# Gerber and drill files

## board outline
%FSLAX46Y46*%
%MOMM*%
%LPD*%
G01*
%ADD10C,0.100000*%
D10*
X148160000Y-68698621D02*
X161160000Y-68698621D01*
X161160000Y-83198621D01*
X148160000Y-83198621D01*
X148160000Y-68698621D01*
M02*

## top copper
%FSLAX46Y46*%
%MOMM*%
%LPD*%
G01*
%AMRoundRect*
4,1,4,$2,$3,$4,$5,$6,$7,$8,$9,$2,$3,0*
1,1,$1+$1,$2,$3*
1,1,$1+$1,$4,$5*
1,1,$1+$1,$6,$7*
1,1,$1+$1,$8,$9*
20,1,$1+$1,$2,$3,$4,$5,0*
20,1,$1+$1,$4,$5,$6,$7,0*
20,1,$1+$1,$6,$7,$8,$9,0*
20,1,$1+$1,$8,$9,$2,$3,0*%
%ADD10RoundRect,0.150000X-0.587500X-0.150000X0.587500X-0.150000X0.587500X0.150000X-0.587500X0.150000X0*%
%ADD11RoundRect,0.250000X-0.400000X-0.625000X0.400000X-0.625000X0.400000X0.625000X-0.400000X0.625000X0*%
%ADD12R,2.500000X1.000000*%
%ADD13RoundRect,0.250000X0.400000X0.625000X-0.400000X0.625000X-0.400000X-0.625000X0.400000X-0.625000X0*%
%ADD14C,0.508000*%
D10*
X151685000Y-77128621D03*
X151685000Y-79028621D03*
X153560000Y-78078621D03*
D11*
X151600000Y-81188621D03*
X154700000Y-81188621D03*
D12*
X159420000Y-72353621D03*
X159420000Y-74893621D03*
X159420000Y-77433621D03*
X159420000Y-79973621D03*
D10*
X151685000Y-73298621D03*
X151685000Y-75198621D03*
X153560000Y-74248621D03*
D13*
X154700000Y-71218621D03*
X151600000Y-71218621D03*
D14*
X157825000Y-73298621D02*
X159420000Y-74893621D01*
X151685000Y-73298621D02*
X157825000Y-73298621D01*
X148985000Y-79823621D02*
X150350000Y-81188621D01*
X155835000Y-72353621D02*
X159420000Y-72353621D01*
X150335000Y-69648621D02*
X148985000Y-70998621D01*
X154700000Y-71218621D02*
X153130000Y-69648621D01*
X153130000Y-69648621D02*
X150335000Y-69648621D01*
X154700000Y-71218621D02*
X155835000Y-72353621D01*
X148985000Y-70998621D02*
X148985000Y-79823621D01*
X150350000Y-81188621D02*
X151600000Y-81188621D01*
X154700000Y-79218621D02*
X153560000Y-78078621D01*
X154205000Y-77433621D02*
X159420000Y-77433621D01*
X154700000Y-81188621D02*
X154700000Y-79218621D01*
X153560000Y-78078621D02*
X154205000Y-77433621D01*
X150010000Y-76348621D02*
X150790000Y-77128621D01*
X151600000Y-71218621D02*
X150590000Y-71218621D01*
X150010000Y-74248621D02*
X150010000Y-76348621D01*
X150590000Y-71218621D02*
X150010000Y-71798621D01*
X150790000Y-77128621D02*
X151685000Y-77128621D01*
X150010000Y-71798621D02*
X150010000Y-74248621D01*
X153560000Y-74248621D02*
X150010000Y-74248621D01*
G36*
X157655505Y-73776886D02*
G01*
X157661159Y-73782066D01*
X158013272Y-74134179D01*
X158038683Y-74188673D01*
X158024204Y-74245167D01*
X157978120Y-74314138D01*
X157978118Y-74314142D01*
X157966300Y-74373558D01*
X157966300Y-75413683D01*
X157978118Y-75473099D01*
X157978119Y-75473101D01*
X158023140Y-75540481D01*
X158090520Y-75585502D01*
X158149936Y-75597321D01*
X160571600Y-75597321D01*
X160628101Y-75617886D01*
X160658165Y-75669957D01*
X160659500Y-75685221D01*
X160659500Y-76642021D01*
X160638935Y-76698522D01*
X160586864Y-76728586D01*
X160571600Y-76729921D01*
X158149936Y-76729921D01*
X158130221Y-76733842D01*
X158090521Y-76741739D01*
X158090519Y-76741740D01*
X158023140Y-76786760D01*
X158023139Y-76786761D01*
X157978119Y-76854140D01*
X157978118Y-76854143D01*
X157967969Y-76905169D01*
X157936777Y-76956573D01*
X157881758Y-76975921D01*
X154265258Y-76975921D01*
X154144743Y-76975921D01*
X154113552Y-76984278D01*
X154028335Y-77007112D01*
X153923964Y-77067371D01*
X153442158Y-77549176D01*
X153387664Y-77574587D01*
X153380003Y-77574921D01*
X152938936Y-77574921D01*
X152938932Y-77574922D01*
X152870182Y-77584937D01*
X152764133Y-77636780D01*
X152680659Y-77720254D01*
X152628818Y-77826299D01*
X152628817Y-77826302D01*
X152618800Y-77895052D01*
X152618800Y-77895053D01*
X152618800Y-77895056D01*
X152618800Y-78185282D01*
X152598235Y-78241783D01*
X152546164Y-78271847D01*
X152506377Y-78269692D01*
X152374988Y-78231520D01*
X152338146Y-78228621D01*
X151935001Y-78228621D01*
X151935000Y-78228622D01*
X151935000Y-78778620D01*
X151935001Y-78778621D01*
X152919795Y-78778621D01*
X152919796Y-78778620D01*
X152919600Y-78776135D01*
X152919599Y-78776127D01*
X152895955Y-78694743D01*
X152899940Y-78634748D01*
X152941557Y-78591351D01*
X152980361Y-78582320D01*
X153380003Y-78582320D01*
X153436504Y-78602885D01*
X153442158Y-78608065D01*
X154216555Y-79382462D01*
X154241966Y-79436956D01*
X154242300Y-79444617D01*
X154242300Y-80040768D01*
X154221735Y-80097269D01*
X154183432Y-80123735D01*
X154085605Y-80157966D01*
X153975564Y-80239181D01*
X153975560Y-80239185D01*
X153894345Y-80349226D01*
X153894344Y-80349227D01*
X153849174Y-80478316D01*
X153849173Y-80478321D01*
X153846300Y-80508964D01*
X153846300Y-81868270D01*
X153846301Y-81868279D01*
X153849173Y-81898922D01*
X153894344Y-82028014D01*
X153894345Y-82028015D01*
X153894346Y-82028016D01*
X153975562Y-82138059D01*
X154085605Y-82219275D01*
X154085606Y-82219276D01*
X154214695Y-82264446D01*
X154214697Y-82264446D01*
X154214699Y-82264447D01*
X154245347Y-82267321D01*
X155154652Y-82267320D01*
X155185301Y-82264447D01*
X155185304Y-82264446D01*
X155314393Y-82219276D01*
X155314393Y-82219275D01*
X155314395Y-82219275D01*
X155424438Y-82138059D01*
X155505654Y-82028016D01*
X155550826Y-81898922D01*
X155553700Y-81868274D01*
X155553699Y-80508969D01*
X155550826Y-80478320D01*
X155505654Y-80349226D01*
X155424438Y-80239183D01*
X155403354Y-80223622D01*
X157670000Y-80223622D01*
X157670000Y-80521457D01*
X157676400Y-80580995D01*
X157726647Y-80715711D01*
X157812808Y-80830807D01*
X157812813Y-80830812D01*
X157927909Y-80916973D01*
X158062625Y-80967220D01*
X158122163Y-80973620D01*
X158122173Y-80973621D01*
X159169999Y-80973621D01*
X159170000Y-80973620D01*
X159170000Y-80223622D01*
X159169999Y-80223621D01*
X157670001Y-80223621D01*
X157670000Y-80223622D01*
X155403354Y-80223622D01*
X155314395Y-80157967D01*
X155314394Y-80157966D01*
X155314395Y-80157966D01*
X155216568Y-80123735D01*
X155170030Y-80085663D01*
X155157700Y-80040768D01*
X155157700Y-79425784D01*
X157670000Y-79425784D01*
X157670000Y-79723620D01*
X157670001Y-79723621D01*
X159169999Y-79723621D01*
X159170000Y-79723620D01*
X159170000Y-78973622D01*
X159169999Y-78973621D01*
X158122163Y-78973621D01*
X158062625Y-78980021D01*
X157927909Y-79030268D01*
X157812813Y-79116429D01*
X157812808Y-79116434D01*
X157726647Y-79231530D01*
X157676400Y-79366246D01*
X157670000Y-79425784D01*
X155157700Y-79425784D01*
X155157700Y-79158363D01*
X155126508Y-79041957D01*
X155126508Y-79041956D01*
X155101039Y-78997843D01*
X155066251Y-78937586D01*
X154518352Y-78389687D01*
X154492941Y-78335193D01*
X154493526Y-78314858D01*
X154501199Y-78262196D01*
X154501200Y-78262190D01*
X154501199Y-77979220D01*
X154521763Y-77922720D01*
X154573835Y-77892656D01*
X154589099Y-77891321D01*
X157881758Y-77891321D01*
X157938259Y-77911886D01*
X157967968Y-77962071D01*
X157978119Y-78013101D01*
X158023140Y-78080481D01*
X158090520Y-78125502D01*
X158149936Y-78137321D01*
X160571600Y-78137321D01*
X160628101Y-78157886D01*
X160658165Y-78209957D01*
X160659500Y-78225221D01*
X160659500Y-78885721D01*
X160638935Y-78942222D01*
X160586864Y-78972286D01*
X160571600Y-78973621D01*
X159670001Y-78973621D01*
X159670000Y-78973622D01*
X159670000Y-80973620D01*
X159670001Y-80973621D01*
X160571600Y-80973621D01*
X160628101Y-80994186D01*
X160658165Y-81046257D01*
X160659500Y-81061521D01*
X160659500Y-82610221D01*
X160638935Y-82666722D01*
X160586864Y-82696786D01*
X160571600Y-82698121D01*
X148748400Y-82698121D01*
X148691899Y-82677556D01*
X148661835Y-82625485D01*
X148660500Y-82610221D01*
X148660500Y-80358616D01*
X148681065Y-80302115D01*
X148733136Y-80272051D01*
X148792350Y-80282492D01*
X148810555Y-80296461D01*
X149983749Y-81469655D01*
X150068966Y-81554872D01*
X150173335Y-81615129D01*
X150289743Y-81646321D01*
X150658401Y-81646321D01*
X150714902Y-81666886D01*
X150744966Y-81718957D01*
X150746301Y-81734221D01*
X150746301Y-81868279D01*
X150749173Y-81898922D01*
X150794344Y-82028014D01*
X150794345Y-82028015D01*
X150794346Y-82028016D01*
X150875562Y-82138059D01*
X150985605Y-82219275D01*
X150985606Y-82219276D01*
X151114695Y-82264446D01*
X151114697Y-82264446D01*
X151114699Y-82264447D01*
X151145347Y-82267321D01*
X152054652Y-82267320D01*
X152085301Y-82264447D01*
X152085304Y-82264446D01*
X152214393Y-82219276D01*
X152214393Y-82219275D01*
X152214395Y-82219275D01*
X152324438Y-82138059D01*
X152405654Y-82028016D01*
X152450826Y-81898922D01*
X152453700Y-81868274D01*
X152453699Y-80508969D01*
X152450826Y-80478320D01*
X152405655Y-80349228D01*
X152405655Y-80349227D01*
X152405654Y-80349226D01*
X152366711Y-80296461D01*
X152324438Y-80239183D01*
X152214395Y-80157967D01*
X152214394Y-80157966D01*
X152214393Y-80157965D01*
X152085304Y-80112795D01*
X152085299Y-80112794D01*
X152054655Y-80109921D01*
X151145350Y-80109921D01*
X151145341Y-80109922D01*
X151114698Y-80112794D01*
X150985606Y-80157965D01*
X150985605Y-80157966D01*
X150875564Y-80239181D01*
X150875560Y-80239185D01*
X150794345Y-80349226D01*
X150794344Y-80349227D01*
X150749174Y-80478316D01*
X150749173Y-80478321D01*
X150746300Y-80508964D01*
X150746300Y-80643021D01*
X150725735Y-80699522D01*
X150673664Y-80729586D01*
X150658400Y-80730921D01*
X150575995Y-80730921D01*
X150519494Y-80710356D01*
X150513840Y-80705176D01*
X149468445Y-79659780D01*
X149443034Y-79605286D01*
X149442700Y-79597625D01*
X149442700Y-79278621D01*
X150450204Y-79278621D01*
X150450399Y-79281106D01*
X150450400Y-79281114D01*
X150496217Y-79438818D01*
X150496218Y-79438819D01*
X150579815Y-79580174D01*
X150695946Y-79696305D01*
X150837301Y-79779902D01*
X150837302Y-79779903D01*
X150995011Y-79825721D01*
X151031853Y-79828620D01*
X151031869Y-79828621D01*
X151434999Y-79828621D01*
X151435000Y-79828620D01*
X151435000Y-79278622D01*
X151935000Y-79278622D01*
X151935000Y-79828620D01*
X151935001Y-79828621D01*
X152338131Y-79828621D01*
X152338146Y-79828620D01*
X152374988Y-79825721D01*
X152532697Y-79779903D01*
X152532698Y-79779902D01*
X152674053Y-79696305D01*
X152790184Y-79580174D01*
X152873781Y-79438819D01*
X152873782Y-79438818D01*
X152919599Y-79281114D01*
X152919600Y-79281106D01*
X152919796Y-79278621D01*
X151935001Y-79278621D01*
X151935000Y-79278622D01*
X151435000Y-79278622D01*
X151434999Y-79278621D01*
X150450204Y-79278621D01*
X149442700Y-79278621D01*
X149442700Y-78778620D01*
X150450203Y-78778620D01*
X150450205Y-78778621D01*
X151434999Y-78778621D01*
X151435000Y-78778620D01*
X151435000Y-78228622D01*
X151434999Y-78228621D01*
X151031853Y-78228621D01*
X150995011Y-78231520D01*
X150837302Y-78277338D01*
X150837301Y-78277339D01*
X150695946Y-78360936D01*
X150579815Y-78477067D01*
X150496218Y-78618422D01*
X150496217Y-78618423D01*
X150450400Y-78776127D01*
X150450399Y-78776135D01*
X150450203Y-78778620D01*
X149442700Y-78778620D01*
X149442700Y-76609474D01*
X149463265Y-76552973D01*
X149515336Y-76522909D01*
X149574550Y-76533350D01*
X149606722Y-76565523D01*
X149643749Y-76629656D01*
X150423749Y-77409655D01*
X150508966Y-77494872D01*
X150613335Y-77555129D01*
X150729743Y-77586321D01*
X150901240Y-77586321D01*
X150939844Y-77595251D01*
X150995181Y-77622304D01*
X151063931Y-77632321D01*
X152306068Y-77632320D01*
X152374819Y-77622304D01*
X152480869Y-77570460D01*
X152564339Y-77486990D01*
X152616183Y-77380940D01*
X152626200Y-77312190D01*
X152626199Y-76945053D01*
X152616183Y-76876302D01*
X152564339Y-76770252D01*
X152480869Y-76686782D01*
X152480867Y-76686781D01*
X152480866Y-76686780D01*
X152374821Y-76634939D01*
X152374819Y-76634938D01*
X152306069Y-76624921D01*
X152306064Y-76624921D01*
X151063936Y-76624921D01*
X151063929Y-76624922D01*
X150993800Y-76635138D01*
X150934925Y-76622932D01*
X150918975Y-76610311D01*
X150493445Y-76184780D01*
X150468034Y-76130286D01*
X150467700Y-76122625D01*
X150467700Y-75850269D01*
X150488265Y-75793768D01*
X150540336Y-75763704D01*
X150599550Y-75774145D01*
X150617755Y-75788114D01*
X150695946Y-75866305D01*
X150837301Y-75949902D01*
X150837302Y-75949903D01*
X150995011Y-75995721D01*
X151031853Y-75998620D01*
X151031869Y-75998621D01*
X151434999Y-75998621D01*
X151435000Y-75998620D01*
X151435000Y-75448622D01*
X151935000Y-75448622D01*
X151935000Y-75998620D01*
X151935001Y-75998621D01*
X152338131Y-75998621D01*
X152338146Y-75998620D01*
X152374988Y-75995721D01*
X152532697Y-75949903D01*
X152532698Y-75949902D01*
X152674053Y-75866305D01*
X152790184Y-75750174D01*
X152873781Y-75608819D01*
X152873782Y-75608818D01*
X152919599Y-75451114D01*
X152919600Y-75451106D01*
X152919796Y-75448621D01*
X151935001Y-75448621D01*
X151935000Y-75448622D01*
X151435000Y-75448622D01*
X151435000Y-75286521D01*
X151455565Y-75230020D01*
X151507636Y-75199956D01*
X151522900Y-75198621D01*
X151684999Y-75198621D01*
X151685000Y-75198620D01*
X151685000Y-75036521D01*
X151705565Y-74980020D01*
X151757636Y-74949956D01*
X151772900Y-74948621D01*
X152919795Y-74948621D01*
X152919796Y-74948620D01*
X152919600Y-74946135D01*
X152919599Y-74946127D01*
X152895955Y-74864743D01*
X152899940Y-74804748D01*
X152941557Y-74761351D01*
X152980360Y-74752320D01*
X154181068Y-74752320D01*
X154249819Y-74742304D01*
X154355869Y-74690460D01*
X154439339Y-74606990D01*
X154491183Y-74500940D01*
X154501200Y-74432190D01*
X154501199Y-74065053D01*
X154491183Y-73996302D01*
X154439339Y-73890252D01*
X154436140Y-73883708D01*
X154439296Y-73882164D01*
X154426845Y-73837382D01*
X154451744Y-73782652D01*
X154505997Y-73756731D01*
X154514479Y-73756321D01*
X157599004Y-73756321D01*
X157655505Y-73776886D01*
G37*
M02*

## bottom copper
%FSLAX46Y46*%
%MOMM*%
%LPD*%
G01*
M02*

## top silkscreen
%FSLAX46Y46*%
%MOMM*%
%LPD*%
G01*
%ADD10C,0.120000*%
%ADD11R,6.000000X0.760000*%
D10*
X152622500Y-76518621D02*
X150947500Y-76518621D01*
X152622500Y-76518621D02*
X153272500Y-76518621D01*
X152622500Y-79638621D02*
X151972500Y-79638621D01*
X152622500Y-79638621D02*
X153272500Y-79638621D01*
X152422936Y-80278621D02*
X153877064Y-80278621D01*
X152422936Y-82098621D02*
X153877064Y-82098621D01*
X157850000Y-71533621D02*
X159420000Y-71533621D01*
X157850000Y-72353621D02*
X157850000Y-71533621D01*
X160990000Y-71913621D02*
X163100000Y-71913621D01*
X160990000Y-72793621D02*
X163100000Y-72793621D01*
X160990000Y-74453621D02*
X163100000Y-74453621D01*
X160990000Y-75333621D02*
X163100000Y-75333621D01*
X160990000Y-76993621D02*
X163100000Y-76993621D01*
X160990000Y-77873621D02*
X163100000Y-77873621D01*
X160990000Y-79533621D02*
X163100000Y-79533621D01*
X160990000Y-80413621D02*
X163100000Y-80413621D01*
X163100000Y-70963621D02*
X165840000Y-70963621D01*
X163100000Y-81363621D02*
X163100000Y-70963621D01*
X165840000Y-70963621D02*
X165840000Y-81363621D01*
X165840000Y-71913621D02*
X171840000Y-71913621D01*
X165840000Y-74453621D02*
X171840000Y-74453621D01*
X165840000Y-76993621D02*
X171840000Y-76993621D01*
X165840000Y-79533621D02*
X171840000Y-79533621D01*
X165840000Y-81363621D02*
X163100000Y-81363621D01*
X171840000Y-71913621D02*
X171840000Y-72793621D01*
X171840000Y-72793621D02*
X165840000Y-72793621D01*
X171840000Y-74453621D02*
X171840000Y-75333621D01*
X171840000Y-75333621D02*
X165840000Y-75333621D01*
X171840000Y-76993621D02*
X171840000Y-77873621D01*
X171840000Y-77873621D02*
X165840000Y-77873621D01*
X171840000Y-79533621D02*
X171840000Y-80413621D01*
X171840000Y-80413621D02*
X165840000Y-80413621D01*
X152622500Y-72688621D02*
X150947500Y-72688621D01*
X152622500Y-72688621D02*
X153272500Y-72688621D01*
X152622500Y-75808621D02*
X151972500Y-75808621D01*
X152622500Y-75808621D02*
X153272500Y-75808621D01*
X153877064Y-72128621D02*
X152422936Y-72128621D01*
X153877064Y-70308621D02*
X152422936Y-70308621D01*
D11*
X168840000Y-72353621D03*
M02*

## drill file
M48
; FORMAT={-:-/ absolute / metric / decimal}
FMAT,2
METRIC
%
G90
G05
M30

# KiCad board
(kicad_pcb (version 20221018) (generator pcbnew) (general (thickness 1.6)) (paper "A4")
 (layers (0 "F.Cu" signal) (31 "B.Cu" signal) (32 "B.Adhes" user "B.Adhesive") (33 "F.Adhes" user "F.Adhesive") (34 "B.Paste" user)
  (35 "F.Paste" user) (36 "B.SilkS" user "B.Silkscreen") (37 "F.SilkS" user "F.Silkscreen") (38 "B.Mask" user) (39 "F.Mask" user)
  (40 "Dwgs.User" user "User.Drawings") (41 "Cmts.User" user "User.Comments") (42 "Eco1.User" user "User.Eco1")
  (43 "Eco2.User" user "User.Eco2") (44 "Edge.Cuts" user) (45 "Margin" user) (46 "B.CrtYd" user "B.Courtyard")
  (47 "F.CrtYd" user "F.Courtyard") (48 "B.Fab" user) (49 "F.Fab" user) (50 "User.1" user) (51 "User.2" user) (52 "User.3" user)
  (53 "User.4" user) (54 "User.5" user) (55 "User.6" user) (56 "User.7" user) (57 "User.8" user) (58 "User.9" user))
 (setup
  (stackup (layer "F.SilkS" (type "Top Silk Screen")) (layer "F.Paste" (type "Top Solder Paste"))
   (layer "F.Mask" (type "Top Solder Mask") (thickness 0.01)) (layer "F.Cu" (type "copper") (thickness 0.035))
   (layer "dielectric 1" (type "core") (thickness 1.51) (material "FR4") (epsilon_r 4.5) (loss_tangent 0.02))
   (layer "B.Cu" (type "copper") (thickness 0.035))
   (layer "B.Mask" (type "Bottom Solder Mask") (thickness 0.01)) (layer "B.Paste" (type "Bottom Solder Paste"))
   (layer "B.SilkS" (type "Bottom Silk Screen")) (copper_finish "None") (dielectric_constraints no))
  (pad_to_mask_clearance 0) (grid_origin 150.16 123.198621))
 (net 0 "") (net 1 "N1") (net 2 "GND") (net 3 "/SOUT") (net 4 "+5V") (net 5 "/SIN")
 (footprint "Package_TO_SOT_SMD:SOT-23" (layer "F.Cu") (at 152.6225 78.078621)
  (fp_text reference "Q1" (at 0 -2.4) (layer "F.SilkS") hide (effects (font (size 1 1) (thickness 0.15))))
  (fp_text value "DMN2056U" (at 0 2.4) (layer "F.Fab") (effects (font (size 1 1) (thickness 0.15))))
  (fp_line (start 0 -1.56) (end -1.675 -1.56) (stroke (width 0.12) (type solid)) (layer "F.SilkS"))
  (fp_line (start 0 -1.56) (end 0.65 -1.56) (stroke (width 0.12) (type solid)) (layer "F.SilkS"))
  (fp_line (start 0 1.56) (end -0.65 1.56) (stroke (width 0.12) (type solid)) (layer "F.SilkS"))
  (fp_line (start 0 1.56) (end 0.65 1.56) (stroke (width 0.12) (type solid)) (layer "F.SilkS"))
  (pad "1" smd roundrect (at -0.9375 -0.95) (size 1.475 0.6) (layers "F.Cu" "F.Paste" "F.Mask") (roundrect_rratio 0.25) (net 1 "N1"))
  (pad "2" smd roundrect (at -0.9375 0.95) (size 1.475 0.6) (layers "F.Cu" "F.Paste" "F.Mask") (roundrect_rratio 0.25) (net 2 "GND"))
  (pad "3" smd roundrect (at 0.9375 0) (size 1.475 0.6) (layers "F.Cu" "F.Paste" "F.Mask") (roundrect_rratio 0.25) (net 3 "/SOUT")))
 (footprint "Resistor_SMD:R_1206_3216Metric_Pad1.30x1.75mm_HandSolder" (layer "F.Cu") (at 153.15 81.188621)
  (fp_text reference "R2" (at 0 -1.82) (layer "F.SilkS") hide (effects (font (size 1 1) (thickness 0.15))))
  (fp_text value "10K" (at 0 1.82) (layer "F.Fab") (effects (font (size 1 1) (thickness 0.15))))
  (fp_line (start -0.727064 -0.91) (end 0.727064 -0.91) (stroke (width 0.12) (type solid)) (layer "F.SilkS"))
  (fp_line (start -0.727064 0.91) (end 0.727064 0.91) (stroke (width 0.12) (type solid)) (layer "F.SilkS"))
  (pad "1" smd roundrect (at -1.55 0) (size 1.3 1.75) (layers "F.Cu" "F.Paste" "F.Mask") (roundrect_rratio 0.1923076923) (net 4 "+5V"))
  (pad "2" smd roundrect (at 1.55 0) (size 1.3 1.75) (layers "F.Cu" "F.Paste" "F.Mask") (roundrect_rratio 0.1923076923) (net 3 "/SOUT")))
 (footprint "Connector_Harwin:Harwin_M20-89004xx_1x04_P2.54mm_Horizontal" (layer "F.Cu") (at 164.945 76.163621)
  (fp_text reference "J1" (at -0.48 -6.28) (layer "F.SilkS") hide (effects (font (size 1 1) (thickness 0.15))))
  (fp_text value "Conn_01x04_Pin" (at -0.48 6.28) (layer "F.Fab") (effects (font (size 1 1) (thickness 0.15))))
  (fp_line (start -7.095 -4.63) (end -5.525 -4.63) (stroke (width 0.12) (type solid)) (layer "F.SilkS"))
  (fp_line (start -7.095 -3.81) (end -7.095 -4.63) (stroke (width 0.12) (type solid)) (layer "F.SilkS"))
  (fp_line (start -3.955 -4.25) (end -1.845 -4.25) (stroke (width 0.12) (type solid)) (layer "F.SilkS"))
  (fp_line (start -3.955 -3.37) (end -1.845 -3.37) (stroke (width 0.12) (type solid)) (layer "F.SilkS"))
  (fp_line (start -3.955 -1.71) (end -1.845 -1.71) (stroke (width 0.12) (type solid)) (layer "F.SilkS"))
  (fp_line (start -3.955 -0.83) (end -1.845 -0.83) (stroke (width 0.12) (type solid)) (layer "F.SilkS"))
  (fp_line (start -3.955 0.83) (end -1.845 0.83) (stroke (width 0.12) (type solid)) (layer "F.SilkS"))
  (fp_line (start -3.955 1.71) (end -1.845 1.71) (stroke (width 0.12) (type solid)) (layer "F.SilkS"))
  (fp_line (start -3.955 3.37) (end -1.845 3.37) (stroke (width 0.12) (type solid)) (layer "F.SilkS"))
  (fp_line (start -3.955 4.25) (end -1.845 4.25) (stroke (width 0.12) (type solid)) (layer "F.SilkS"))
  (fp_line (start -1.845 -5.2) (end 0.895 -5.2) (stroke (width 0.12) (type solid)) (layer "F.SilkS"))
  (fp_line (start -1.845 5.2) (end -1.845 -5.2) (stroke (width 0.12) (type solid)) (layer "F.SilkS"))
  (fp_line (start 0.895 -5.2) (end 0.895 5.2) (stroke (width 0.12) (type solid)) (layer "F.SilkS"))
  (fp_line (start 0.895 -4.25) (end 6.895 -4.25) (stroke (width 0.12) (type solid)) (layer "F.SilkS"))
  (fp_line (start 0.895 -1.71) (end 6.895 -1.71) (stroke (width 0.12) (type solid)) (layer "F.SilkS"))
  (fp_line (start 0.895 0.83) (end 6.895 0.83) (stroke (width 0.12) (type solid)) (layer "F.SilkS"))
  (fp_line (start 0.895 3.37) (end 6.895 3.37) (stroke (width 0.12) (type solid)) (layer "F.SilkS"))
  (fp_line (start 0.895 5.2) (end -1.845 5.2) (stroke (width 0.12) (type solid)) (layer "F.SilkS"))
  (fp_line (start 6.895 -4.25) (end 6.895 -3.37) (stroke (width 0.12) (type solid)) (layer "F.SilkS"))
  (fp_line (start 6.895 -3.37) (end 0.895 -3.37) (stroke (width 0.12) (type solid)) (layer "F.SilkS"))
  (fp_line (start 6.895 -1.71) (end 6.895 -0.83) (stroke (width 0.12) (type solid)) (layer "F.SilkS"))
  (fp_line (start 6.895 -0.83) (end 0.895 -0.83) (stroke (width 0.12) (type solid)) (layer "F.SilkS"))
  (fp_line (start 6.895 0.83) (end 6.895 1.71) (stroke (width 0.12) (type solid)) (layer "F.SilkS"))
  (fp_line (start 6.895 1.71) (end 0.895 1.71) (stroke (width 0.12) (type solid)) (layer "F.SilkS"))
  (fp_line (start 6.895 3.37) (end 6.895 4.25) (stroke (width 0.12) (type solid)) (layer "F.SilkS"))
  (fp_line (start 6.895 4.25) (end 0.895 4.25) (stroke (width 0.12) (type solid)) (layer "F.SilkS"))
  (pad "" smd rect (at 3.895 -3.81) (size 6 0.76) (layers "F.SilkS"))
  (pad "1" smd rect (at -5.525 -3.81) (size 2.5 1) (layers "F.Cu" "F.Paste" "F.Mask") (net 4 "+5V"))
  (pad "2" smd rect (at -5.525 -1.27) (size 2.5 1) (layers "F.Cu" "F.Paste" "F.Mask") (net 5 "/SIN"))
  (pad "3" smd rect (at -5.525 1.27) (size 2.5 1) (layers "F.Cu" "F.Paste" "F.Mask") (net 3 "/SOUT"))
  (pad "4" smd rect (at -5.525 3.81) (size 2.5 1) (layers "F.Cu" "F.Paste" "F.Mask") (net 2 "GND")))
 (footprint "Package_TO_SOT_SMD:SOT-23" (layer "F.Cu") (at 152.6225 74.248621)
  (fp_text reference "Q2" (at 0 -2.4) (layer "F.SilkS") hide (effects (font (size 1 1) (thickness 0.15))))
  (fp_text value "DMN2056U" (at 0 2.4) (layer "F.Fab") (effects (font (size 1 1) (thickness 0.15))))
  (fp_line (start 0 -1.56) (end -1.675 -1.56) (stroke (width 0.12) (type solid)) (layer "F.SilkS"))
  (fp_line (start 0 -1.56) (end 0.65 -1.56) (stroke (width 0.12) (type solid)) (layer "F.SilkS"))
  (fp_line (start 0 1.56) (end -0.65 1.56) (stroke (width 0.12) (type solid)) (layer "F.SilkS"))
  (fp_line (start 0 1.56) (end 0.65 1.56) (stroke (width 0.12) (type solid)) (layer "F.SilkS"))
  (pad "1" smd roundrect (at -0.9375 -0.95) (size 1.475 0.6) (layers "F.Cu" "F.Paste" "F.Mask") (roundrect_rratio 0.25) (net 5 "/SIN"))
  (pad "2" smd roundrect (at -0.9375 0.95) (size 1.475 0.6) (layers "F.Cu" "F.Paste" "F.Mask") (roundrect_rratio 0.25) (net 2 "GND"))
  (pad "3" smd roundrect (at 0.9375 0) (size 1.475 0.6) (layers "F.Cu" "F.Paste" "F.Mask") (roundrect_rratio 0.25) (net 1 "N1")))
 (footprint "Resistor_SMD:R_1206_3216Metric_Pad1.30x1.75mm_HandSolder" (layer "F.Cu") (at 153.15 71.218621 180)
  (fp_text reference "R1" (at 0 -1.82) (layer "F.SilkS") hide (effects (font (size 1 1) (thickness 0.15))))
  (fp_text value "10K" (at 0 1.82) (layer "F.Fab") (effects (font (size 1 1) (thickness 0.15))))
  (fp_line (start -0.727064 -0.91) (end 0.727064 -0.91) (stroke (width 0.12) (type solid)) (layer "F.SilkS"))
  (fp_line (start -0.727064 0.91) (end 0.727064 0.91) (stroke (width 0.12) (type solid)) (layer "F.SilkS"))
  (pad "1" smd roundrect (at -1.55 0 180) (size 1.3 1.75) (layers "F.Cu" "F.Paste" "F.Mask") (roundrect_rratio 0.1923076923) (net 4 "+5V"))
  (pad "2" smd roundrect (at 1.55 0 180) (size 1.3 1.75) (layers "F.Cu" "F.Paste" "F.Mask") (roundrect_rratio 0.1923076923) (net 1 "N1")))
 (gr_rect (start 148.16 68.698621) (end 161.16 83.198621) (stroke (width 0.1) (type default)) (fill none) (layer "Edge.Cuts"))
 (segment (start 157.825 73.298621) (end 159.42 74.893621) (width 0.508) (layer "F.Cu") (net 5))
 (segment (start 151.685 73.298621) (end 157.825 73.298621) (width 0.508) (layer "F.Cu") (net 5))
 (segment (start 148.985 79.823621) (end 150.35 81.188621) (width 0.508) (layer "F.Cu") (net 4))
 (segment (start 155.835 72.353621) (end 159.42 72.353621) (width 0.508) (layer "F.Cu") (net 4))
 (segment (start 150.335 69.648621) (end 148.985 70.998621) (width 0.508) (layer "F.Cu") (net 4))
 (segment (start 154.7 71.218621) (end 153.13 69.648621) (width 0.508) (layer "F.Cu") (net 4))
 (segment (start 153.13 69.648621) (end 150.335 69.648621) (width 0.508) (layer "F.Cu") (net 4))
 (segment (start 154.7 71.218621) (end 155.835 72.353621) (width 0.508) (layer "F.Cu") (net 4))
 (segment (start 148.985 70.998621) (end 148.985 79.823621) (width 0.508) (layer "F.Cu") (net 4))
 (segment (start 150.35 81.188621) (end 151.6 81.188621) (width 0.508) (layer "F.Cu") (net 4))
 (segment (start 154.7 79.218621) (end 153.56 78.078621) (width 0.508) (layer "F.Cu") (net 3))
 (segment (start 154.205 77.433621) (end 159.42 77.433621) (width 0.508) (layer "F.Cu") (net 3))
 (segment (start 154.7 81.188621) (end 154.7 79.218621) (width 0.508) (layer "F.Cu") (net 3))
 (segment (start 153.56 78.078621) (end 154.205 77.433621) (width 0.508) (layer "F.Cu") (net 3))
 (segment (start 150.01 76.348621) (end 150.79 77.128621) (width 0.508) (layer "F.Cu") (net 1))
 (segment (start 151.6 71.218621) (end 150.59 71.218621) (width 0.508) (layer "F.Cu") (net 1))
 (segment (start 150.01 74.248621) (end 150.01 76.348621) (width 0.508) (layer "F.Cu") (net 1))
 (segment (start 150.59 71.218621) (end 150.01 71.798621) (width 0.508) (layer "F.Cu") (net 1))
 (segment (start 150.79 77.128621) (end 151.685 77.128621) (width 0.508) (layer "F.Cu") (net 1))
 (segment (start 150.01 71.798621) (end 150.01 74.248621) (width 0.508) (layer "F.Cu") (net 1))
 (segment (start 153.56 74.248621) (end 150.01 74.248621) (width 0.508) (layer "F.Cu") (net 1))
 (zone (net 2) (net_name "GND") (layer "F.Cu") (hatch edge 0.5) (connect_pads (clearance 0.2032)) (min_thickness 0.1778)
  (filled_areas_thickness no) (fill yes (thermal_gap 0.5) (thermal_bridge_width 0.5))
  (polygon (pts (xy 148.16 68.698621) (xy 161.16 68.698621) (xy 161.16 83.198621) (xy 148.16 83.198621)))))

